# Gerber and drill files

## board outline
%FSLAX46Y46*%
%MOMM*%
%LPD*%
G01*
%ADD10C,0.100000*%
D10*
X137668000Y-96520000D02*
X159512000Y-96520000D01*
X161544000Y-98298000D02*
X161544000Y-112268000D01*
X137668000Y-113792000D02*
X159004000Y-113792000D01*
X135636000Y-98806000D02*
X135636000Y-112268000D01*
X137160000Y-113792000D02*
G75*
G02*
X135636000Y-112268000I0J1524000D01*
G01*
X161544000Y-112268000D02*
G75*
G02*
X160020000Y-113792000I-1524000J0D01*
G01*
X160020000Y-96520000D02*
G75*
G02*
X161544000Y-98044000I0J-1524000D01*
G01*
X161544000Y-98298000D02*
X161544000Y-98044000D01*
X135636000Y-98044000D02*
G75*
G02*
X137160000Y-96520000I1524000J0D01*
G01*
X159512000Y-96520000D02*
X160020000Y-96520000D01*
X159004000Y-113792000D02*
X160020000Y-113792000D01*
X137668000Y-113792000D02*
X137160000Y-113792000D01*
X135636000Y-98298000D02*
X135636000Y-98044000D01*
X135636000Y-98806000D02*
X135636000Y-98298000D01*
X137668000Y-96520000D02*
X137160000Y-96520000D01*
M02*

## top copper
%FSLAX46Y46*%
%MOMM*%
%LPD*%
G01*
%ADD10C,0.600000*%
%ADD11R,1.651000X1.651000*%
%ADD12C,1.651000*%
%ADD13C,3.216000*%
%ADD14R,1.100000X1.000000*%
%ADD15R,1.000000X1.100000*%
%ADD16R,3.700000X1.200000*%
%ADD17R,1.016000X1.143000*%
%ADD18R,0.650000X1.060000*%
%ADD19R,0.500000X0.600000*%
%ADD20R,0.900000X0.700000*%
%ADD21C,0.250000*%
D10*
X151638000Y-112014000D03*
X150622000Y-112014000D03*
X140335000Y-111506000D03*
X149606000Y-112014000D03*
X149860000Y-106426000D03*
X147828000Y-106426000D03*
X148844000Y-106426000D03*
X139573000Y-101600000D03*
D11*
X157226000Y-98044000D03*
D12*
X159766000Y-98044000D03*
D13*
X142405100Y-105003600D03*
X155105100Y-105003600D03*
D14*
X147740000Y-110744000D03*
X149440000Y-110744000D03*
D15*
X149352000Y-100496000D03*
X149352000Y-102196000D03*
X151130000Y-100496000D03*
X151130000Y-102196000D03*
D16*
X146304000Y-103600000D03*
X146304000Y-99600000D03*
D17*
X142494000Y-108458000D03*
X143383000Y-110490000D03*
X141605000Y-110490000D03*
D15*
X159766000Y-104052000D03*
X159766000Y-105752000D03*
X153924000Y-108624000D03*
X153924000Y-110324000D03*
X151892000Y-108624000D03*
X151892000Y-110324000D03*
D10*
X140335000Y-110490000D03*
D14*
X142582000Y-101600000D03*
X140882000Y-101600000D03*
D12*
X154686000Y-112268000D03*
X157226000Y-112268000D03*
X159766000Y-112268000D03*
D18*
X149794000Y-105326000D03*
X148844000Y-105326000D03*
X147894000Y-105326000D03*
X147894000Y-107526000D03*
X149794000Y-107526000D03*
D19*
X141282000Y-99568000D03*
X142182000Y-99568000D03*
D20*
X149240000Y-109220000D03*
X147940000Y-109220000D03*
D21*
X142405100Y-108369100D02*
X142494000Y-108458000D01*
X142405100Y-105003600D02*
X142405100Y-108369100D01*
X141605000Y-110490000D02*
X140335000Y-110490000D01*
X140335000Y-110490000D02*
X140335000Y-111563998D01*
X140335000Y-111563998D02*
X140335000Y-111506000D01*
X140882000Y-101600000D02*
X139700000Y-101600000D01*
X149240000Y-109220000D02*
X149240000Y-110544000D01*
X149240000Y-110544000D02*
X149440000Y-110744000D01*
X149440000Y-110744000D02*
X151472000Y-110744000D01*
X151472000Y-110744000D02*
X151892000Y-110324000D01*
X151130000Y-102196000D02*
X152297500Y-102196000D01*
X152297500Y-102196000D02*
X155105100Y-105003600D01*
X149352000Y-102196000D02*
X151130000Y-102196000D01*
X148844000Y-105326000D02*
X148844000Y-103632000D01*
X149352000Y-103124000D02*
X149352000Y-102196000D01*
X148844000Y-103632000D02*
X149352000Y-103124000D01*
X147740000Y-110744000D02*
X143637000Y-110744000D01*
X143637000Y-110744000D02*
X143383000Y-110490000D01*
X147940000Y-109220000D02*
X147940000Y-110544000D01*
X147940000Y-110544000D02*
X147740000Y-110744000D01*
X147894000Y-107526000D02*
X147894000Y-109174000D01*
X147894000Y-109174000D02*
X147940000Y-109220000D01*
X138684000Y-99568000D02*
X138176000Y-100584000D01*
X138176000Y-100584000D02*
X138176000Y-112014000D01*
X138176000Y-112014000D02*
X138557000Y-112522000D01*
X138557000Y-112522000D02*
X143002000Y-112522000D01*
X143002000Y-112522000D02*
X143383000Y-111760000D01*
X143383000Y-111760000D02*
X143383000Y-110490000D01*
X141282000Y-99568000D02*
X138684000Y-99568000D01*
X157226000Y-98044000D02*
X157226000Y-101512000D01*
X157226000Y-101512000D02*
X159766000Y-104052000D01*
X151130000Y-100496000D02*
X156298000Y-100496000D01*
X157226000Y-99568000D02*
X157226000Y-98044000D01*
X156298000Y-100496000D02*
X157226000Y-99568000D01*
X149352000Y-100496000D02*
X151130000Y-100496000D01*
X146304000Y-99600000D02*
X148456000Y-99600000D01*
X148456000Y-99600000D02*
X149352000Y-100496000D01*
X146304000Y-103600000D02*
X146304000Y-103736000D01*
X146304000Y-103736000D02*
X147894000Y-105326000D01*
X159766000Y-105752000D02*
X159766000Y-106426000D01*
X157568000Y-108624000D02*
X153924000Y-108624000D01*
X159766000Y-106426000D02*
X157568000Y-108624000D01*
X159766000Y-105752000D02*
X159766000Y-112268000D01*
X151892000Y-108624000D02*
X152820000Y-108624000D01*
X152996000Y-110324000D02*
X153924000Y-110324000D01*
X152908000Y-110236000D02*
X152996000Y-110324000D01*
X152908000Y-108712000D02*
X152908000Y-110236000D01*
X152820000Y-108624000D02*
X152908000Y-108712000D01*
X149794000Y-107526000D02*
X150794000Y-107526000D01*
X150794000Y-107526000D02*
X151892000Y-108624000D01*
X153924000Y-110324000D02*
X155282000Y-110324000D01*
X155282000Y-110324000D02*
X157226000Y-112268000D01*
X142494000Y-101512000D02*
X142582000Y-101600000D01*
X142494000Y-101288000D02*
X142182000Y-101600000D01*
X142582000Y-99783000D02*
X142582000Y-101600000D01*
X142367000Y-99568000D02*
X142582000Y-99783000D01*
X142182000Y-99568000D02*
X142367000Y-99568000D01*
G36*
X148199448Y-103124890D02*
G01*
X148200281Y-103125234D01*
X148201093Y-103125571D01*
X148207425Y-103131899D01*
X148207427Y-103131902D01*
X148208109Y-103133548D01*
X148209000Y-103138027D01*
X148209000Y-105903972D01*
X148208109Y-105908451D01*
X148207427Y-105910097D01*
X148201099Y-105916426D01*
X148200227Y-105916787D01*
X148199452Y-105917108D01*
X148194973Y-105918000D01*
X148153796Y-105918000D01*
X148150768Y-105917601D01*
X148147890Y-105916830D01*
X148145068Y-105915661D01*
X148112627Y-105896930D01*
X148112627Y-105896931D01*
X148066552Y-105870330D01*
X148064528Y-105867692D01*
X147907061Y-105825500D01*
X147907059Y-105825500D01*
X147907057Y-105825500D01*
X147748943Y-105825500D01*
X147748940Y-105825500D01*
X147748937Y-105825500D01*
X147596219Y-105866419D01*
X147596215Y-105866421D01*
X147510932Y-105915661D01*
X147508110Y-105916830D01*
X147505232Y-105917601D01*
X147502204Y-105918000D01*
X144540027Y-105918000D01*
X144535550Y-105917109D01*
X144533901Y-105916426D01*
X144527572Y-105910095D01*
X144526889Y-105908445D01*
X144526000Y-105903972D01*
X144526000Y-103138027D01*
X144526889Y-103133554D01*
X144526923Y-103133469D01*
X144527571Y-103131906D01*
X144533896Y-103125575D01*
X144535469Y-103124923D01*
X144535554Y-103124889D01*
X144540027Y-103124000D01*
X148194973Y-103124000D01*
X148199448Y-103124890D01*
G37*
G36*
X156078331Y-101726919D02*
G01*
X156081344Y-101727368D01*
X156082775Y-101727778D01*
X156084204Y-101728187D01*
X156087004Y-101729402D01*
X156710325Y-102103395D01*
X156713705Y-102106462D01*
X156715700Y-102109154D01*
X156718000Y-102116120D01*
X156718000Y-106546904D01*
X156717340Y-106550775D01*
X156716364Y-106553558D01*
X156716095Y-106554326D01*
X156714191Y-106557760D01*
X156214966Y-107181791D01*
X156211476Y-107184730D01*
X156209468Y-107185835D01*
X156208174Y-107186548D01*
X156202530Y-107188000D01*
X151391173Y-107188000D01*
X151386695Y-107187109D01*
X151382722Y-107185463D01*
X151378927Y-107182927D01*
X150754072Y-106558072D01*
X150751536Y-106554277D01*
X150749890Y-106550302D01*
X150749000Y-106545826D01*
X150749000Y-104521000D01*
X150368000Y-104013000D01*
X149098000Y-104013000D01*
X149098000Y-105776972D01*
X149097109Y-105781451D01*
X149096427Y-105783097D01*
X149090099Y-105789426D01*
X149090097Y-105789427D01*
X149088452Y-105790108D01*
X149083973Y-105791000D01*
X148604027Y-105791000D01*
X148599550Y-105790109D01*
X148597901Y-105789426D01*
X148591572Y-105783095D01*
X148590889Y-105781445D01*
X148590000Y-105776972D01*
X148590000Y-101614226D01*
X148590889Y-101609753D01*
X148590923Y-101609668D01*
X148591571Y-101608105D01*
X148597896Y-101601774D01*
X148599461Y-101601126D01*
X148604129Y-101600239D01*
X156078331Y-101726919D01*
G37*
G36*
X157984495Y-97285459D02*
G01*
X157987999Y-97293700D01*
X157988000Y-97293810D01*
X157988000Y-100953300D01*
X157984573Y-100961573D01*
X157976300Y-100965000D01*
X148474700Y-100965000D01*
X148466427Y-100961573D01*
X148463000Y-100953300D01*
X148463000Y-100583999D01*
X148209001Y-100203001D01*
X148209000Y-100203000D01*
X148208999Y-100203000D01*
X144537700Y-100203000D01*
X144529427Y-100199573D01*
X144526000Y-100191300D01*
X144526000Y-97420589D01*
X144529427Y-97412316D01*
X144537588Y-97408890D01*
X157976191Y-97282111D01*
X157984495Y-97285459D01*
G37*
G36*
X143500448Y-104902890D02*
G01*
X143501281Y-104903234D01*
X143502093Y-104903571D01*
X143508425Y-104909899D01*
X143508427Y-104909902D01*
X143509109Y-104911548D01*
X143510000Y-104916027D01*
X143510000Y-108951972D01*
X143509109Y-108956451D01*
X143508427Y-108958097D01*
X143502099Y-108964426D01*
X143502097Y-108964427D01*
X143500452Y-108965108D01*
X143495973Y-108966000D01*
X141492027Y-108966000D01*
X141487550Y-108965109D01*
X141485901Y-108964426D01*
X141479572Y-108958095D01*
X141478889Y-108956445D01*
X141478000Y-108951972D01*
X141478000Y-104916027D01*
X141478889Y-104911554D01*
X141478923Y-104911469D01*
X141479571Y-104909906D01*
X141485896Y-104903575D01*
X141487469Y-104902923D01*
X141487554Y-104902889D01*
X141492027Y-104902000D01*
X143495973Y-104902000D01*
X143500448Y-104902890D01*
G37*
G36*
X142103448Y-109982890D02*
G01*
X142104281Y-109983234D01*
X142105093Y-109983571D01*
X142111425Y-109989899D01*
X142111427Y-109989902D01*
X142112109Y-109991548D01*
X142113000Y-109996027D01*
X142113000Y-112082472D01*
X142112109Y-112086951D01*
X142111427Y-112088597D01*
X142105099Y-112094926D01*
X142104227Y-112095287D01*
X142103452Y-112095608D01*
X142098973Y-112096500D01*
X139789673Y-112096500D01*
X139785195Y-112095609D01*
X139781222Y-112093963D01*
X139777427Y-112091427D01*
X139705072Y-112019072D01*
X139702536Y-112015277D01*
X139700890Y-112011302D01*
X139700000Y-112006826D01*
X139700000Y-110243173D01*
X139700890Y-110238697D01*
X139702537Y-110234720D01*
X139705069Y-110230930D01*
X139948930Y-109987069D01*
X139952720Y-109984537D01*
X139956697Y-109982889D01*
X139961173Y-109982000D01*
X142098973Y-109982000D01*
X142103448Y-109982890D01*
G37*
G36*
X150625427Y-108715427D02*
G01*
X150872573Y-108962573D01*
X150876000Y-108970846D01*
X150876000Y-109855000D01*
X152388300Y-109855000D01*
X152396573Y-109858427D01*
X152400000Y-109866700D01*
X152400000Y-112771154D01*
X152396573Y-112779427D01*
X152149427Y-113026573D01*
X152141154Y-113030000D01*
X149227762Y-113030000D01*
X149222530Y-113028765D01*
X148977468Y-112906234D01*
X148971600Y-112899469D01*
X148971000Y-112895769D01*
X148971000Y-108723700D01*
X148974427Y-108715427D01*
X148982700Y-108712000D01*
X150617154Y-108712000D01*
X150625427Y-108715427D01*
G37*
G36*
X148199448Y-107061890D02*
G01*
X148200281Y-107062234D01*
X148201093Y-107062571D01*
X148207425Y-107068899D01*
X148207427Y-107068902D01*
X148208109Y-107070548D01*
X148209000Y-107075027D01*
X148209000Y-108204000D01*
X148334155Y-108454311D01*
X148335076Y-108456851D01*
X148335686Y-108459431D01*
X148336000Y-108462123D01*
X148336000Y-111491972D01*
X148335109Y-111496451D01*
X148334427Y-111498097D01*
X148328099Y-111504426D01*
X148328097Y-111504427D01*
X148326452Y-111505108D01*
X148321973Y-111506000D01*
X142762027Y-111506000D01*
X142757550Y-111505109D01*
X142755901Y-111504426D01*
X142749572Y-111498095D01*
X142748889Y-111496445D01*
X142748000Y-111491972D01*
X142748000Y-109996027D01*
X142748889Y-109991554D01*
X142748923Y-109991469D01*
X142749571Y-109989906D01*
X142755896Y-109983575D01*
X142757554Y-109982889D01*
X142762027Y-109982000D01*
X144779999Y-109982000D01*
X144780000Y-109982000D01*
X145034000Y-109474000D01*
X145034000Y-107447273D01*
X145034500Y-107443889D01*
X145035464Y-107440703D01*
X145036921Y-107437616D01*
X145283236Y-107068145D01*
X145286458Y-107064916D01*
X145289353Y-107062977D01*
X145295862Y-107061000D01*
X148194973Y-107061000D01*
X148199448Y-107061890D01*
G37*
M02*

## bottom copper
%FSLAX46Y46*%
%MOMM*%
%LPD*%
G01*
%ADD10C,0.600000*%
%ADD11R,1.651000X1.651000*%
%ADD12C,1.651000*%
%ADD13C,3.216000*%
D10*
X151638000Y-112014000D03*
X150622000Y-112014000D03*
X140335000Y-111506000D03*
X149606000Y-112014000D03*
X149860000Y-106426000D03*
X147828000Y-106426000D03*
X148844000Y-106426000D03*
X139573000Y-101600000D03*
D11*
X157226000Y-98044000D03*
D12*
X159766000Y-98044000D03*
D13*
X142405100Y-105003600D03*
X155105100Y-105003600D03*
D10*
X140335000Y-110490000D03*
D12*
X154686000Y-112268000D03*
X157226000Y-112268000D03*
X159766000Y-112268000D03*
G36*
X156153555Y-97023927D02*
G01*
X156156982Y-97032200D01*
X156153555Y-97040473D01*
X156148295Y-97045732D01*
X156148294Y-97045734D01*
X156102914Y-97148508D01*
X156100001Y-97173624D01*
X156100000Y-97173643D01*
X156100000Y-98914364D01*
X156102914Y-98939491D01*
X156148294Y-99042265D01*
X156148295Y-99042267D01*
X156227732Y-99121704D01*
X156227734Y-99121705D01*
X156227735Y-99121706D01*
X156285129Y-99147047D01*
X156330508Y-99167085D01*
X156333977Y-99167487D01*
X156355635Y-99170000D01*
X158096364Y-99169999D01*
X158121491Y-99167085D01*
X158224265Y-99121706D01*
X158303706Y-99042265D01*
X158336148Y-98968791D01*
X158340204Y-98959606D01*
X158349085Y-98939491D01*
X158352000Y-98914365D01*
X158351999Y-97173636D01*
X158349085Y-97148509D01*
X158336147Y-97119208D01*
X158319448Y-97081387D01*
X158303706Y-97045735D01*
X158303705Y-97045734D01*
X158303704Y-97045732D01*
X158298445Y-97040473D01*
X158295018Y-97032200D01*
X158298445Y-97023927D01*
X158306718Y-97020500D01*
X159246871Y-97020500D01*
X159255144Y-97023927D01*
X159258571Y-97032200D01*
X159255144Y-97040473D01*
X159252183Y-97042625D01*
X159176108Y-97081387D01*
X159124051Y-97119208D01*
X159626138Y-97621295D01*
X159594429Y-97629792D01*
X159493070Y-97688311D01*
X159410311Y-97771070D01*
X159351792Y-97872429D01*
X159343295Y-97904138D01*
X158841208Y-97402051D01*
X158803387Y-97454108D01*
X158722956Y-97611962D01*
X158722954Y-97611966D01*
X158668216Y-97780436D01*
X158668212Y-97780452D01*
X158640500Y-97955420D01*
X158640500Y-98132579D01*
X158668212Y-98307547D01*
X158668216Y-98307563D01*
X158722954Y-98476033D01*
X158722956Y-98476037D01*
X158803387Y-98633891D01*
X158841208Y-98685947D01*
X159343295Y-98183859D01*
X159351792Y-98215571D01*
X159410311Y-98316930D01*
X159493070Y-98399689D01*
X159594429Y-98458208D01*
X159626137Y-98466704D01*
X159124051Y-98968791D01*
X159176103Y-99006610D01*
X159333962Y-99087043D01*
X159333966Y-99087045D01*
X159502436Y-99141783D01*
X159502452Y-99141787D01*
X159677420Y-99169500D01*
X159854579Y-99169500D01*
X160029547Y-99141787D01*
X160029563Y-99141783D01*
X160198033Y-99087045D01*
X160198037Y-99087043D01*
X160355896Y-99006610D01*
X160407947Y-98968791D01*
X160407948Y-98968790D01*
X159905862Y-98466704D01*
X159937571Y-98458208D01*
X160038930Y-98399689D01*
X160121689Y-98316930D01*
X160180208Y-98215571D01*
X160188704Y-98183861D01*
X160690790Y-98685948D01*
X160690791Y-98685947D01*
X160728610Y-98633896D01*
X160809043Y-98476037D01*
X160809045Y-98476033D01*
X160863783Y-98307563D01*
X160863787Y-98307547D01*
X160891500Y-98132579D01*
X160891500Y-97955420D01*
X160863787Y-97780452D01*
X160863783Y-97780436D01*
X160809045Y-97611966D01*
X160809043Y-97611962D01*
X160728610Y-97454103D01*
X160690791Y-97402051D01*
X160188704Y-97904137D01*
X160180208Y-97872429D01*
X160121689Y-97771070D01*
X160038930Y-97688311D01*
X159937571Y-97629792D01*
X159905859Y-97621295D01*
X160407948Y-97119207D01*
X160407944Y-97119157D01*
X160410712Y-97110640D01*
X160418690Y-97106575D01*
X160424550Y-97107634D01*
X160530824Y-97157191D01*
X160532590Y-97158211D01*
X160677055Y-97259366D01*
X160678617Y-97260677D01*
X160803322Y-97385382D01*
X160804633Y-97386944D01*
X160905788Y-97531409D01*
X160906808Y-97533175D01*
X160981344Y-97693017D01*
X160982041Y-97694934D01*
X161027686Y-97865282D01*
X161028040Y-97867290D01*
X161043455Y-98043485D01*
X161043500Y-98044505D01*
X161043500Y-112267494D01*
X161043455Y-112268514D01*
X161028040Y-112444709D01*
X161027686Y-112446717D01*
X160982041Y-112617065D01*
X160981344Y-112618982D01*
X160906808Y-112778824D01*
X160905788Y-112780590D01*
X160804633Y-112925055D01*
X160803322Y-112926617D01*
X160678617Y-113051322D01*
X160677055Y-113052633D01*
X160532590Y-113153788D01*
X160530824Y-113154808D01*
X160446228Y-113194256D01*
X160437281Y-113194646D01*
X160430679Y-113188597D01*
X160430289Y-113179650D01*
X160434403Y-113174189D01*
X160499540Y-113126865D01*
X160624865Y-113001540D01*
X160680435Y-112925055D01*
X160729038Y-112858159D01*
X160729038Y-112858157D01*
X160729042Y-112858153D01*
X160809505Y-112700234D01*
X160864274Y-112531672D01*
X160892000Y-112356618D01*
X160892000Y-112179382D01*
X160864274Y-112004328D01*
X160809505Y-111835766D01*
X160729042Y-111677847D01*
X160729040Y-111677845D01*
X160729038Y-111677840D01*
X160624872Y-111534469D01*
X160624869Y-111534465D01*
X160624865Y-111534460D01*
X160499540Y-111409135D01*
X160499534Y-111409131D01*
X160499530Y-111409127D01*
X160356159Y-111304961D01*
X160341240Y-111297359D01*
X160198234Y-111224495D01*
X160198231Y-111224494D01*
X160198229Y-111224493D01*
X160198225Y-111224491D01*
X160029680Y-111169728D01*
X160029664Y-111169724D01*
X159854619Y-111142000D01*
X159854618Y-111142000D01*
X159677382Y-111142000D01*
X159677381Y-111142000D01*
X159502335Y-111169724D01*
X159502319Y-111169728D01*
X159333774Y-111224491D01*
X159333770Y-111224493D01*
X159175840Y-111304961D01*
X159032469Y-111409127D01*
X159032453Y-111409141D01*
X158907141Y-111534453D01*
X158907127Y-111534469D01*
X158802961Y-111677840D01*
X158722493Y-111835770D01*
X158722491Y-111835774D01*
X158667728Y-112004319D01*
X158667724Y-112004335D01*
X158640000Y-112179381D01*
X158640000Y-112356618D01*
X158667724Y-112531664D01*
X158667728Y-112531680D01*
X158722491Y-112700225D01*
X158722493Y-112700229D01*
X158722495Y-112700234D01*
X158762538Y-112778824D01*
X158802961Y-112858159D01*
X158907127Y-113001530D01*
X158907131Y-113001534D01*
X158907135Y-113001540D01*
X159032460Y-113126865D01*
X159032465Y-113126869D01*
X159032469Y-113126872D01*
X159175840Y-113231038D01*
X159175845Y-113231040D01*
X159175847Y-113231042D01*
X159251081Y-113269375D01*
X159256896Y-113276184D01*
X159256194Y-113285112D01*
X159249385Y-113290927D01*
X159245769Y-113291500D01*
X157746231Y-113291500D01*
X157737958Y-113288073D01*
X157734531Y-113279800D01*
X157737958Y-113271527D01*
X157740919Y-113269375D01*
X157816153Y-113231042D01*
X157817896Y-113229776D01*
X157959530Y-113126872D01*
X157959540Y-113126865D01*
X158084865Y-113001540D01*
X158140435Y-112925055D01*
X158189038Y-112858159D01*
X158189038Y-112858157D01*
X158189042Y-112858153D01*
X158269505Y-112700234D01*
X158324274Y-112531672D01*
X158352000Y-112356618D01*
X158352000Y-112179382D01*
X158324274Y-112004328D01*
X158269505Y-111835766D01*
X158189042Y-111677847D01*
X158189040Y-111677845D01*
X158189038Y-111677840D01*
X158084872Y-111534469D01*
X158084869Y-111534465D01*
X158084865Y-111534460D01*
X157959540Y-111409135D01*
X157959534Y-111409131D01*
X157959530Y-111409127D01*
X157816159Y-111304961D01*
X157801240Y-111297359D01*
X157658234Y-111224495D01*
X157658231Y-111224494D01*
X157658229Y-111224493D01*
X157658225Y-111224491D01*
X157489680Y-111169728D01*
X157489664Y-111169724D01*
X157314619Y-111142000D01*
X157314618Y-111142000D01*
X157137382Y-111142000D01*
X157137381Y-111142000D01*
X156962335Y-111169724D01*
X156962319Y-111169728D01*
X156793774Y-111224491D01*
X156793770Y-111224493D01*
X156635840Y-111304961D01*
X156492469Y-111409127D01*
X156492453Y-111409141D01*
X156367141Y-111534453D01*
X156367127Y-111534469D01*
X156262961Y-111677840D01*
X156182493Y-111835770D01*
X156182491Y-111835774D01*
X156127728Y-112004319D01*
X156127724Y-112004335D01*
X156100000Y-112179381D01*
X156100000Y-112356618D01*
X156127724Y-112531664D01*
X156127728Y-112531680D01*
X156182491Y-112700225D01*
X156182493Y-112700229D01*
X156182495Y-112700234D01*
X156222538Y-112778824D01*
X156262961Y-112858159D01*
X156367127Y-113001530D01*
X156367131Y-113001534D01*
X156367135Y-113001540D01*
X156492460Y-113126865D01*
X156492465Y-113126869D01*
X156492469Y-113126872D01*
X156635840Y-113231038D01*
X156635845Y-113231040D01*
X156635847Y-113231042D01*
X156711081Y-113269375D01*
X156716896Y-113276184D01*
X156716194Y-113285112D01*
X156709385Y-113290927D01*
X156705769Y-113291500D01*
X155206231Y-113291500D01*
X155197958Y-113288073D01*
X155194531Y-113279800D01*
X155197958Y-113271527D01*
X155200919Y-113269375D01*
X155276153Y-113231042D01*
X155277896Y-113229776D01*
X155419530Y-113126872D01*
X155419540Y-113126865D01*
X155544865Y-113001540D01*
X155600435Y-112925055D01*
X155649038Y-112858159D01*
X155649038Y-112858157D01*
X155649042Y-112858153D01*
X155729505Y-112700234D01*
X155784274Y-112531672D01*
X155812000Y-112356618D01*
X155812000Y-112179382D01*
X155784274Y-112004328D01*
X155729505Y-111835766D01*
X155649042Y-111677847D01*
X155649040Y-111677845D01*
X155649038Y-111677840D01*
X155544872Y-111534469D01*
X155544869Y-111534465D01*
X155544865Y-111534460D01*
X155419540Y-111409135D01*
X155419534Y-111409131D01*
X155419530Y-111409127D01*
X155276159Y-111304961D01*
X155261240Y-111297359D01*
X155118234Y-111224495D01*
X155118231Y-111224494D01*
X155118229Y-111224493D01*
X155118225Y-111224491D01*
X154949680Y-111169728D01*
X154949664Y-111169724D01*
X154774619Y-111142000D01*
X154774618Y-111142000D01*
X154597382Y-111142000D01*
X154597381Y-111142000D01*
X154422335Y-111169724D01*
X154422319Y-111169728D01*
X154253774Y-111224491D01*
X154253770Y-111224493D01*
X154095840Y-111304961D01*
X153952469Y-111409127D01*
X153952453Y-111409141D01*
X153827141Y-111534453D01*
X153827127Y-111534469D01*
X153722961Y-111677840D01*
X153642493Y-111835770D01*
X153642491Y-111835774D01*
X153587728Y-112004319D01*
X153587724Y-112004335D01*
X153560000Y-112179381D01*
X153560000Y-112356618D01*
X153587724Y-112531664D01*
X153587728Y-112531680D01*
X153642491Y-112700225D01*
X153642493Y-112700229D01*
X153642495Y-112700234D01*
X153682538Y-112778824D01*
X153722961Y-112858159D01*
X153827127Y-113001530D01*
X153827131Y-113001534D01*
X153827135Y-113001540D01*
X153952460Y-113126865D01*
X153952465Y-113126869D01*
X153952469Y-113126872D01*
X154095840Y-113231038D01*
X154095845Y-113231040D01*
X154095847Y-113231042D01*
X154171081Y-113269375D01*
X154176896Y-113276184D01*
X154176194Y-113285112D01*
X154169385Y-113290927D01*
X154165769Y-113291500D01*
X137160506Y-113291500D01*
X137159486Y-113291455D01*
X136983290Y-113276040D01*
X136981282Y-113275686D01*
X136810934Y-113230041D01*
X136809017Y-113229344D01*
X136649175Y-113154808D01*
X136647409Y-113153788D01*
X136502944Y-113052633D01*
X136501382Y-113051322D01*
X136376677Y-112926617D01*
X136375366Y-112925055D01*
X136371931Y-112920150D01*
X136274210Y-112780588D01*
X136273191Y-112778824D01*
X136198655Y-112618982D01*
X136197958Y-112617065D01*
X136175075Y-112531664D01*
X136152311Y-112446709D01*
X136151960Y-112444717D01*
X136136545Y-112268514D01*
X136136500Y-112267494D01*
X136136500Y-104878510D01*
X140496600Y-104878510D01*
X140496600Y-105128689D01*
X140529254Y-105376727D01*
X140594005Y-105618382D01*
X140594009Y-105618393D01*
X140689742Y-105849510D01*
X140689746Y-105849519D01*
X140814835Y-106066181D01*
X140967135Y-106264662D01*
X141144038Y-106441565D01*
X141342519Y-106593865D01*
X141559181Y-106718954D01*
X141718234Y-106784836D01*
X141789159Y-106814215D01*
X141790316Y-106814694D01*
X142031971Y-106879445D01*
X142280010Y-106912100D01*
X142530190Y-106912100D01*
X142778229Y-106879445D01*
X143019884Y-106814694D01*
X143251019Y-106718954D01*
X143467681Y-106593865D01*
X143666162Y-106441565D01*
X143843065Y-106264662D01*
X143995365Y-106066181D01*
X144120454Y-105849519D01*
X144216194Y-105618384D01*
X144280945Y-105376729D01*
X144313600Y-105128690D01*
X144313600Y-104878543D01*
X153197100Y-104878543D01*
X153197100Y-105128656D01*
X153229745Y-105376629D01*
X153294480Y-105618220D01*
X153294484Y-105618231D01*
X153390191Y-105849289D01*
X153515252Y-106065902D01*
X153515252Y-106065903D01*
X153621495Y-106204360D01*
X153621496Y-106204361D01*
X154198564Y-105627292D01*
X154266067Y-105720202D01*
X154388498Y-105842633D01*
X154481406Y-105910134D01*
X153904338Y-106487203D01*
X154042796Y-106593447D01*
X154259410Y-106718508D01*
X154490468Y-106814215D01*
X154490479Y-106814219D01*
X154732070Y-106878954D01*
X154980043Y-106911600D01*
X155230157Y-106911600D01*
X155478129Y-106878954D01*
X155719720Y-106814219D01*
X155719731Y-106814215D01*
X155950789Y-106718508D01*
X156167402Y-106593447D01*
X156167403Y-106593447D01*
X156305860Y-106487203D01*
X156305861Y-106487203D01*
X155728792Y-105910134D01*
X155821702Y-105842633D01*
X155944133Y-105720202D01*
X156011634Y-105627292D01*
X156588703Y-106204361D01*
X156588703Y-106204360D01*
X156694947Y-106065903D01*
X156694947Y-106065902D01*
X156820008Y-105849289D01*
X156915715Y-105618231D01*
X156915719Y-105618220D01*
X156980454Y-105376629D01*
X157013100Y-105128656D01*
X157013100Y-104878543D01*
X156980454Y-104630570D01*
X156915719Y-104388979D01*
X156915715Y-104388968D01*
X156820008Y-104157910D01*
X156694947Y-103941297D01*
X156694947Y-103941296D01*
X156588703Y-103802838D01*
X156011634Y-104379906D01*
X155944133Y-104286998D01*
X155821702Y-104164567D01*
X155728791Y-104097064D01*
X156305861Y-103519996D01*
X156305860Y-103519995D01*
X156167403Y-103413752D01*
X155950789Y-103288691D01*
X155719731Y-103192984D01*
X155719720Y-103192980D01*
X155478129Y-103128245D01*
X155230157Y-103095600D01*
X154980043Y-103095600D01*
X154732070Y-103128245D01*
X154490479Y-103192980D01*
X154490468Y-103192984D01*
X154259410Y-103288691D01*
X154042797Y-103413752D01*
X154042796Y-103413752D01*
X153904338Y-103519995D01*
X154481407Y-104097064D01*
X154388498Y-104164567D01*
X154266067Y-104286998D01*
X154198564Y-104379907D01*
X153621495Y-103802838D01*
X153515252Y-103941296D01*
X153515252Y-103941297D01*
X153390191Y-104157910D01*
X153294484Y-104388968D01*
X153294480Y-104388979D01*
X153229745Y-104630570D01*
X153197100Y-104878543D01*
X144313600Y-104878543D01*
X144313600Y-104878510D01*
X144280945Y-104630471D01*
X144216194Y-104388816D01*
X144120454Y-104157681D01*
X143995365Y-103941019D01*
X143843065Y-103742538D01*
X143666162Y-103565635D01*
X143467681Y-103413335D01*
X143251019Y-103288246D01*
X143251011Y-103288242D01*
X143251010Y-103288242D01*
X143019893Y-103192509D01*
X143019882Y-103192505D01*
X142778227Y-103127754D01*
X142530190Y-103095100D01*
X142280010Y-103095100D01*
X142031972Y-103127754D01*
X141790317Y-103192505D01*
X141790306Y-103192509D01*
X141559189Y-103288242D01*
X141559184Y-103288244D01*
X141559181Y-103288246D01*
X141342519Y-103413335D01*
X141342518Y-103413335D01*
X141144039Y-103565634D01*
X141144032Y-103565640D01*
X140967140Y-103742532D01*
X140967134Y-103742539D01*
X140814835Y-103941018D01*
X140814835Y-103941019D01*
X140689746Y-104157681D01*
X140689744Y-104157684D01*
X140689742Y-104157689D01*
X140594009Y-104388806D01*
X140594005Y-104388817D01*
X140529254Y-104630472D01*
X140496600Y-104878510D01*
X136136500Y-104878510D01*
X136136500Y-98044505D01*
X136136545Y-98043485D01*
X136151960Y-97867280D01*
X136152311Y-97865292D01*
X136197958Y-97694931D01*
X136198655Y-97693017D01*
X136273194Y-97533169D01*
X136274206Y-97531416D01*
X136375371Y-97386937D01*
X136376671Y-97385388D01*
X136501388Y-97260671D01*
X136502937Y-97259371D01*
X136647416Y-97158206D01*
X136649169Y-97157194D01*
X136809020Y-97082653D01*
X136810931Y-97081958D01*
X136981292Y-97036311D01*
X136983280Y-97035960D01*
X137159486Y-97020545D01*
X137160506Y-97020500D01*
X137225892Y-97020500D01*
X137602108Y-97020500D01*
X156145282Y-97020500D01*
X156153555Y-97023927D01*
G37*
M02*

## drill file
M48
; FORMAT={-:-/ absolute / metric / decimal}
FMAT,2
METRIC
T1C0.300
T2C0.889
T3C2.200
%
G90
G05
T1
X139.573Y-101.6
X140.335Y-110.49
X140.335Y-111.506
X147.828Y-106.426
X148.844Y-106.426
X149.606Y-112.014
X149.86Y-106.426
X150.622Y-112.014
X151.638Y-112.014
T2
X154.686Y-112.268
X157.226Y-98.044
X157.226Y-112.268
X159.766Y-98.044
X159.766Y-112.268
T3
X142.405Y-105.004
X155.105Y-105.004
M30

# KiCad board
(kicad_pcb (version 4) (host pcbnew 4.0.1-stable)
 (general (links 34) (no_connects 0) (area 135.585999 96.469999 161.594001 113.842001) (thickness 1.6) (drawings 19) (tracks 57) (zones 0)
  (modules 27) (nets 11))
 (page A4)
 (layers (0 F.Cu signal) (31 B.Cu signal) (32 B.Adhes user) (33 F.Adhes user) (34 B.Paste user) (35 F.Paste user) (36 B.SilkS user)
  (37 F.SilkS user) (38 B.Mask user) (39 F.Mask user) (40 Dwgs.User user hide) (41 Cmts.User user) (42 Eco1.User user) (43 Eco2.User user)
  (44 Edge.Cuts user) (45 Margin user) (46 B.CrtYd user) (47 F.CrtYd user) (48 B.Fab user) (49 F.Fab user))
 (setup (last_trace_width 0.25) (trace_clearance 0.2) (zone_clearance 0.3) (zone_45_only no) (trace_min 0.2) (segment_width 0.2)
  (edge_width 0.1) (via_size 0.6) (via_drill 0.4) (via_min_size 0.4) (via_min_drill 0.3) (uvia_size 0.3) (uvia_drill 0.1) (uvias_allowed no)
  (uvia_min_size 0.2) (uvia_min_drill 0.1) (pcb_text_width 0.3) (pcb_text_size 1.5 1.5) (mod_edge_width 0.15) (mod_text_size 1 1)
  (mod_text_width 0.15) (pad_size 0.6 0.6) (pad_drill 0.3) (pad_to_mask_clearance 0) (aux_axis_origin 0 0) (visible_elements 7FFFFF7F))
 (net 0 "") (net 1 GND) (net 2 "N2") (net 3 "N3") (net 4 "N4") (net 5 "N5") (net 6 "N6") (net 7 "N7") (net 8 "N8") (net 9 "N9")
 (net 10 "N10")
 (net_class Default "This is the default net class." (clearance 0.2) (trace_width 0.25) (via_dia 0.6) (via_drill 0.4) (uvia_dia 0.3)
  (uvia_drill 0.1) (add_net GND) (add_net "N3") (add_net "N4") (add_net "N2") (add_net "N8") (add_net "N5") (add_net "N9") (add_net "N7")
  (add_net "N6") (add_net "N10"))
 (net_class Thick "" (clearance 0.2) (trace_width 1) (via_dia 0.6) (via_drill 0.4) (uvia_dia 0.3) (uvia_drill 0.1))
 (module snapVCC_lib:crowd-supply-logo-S (layer F.Cu) (at 138 98.15 90)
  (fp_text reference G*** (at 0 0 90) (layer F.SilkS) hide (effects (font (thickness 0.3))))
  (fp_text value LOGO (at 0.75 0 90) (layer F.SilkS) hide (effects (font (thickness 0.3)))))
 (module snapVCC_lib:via (layer F.Cu) (at 151.638 112.014)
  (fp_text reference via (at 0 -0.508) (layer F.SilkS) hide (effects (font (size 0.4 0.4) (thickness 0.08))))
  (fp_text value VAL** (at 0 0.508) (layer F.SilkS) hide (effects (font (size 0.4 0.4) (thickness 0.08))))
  (pad 1 thru_hole circle (at 0 0) (size 0.6 0.6) (drill 0.3) (layers *.Cu) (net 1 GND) (zone_connect 2)))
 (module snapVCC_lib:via (layer F.Cu) (at 150.622 112.014)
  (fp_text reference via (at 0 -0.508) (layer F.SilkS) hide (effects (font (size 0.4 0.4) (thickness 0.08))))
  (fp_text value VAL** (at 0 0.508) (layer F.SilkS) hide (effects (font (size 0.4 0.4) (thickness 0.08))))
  (pad 1 thru_hole circle (at 0 0) (size 0.6 0.6) (drill 0.3) (layers *.Cu) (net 1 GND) (zone_connect 2)))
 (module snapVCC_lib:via (layer F.Cu) (at 140.335 111.506)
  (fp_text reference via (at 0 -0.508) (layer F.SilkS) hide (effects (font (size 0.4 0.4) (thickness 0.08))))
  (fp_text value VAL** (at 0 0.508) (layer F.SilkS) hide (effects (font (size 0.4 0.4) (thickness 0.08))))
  (pad 1 thru_hole circle (at 0 0) (size 0.6 0.6) (drill 0.3) (layers *.Cu) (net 1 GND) (zone_connect 2)))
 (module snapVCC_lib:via (layer F.Cu) (at 149.606 112.014)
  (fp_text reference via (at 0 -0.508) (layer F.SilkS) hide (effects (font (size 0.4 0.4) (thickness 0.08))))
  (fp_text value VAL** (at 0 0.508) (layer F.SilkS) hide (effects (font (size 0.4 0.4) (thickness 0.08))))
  (pad 1 thru_hole circle (at 0 0) (size 0.6 0.6) (drill 0.3) (layers *.Cu) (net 1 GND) (zone_connect 2)))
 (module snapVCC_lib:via (layer F.Cu) (at 149.86 106.426)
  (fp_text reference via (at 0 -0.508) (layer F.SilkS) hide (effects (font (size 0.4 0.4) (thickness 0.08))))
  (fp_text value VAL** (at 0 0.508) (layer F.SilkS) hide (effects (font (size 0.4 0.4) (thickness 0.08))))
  (pad 1 thru_hole circle (at 0 0) (size 0.6 0.6) (drill 0.3) (layers *.Cu) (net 1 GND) (zone_connect 2)))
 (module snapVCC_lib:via (layer F.Cu) (at 147.828 106.426)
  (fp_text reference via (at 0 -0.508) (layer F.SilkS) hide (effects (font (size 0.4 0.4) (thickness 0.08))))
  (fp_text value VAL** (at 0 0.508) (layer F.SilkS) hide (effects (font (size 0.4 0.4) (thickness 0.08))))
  (pad 1 thru_hole circle (at 0 0) (size 0.6 0.6) (drill 0.3) (layers *.Cu) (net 1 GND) (zone_connect 2)))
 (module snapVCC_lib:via (layer F.Cu) (at 148.844 106.426)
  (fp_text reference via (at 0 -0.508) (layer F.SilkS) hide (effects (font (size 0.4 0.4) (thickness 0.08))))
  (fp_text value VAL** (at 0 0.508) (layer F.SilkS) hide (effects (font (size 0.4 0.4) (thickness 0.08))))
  (pad 1 thru_hole circle (at 0 0) (size 0.6 0.6) (drill 0.3) (layers *.Cu) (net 1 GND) (zone_connect 2)))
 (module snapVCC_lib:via (layer F.Cu) (at 139.573 101.6)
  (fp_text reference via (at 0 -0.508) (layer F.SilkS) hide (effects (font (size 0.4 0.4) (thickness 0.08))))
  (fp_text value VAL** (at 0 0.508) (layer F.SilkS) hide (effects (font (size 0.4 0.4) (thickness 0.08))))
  (pad 1 thru_hole circle (at 0 0) (size 0.6 0.6) (drill 0.3) (layers *.Cu) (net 1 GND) (zone_connect 2)))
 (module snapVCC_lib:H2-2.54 (layer F.Cu) (at 158.496 98.044 90)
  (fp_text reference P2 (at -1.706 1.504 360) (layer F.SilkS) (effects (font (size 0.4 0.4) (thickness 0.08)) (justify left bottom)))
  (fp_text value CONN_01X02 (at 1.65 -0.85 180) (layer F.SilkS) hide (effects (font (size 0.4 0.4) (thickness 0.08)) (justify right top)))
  (pad 1 thru_hole rect (at 0 -1.27 90) (size 1.651 1.651) (drill 0.889) (layers *.Cu *.Mask) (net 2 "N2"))
  (pad 2 thru_hole circle (at 0 1.27 90) (size 1.651 1.651) (drill 0.889) (layers *.Cu *.Mask) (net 1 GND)))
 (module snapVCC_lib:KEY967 (layer B.Cu) (at 148.7551 105.0036)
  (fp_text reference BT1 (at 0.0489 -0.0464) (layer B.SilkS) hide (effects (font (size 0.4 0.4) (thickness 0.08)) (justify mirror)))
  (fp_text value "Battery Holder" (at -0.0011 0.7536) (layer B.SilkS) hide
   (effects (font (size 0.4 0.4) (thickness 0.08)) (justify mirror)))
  (pad 1 thru_hole circle (at -6.35 0) (size 3.216 3.216) (drill 2.2) (layers *.Cu *.Mask) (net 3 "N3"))
  (pad 2 thru_hole circle (at 6.35 0) (size 3.216 3.216) (drill 2.2) (layers *.Cu *.Mask) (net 1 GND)))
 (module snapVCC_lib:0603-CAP (layer F.Cu) (at 148.59 110.744)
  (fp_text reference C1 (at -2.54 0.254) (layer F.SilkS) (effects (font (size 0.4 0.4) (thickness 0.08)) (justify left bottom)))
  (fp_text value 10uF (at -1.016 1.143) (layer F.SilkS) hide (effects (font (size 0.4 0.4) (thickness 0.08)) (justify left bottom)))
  (pad 1 smd rect (at -0.85 0) (size 1.1 1) (layers F.Cu F.Paste F.Mask) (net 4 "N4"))
  (pad 2 smd rect (at 0.85 0) (size 1.1 1) (layers F.Cu F.Paste F.Mask) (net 1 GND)))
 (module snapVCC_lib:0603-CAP (layer F.Cu) (at 149.352 101.346 270)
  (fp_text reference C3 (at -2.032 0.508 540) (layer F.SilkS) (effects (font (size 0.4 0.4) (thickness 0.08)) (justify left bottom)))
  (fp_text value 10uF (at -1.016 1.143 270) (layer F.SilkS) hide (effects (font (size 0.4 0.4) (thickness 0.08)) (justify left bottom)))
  (pad 1 smd rect (at -0.85 0 270) (size 1.1 1) (layers F.Cu F.Paste F.Mask) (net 2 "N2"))
  (pad 2 smd rect (at 0.85 0 270) (size 1.1 1) (layers F.Cu F.Paste F.Mask) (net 1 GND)))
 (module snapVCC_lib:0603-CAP (layer F.Cu) (at 151.13 101.346 270)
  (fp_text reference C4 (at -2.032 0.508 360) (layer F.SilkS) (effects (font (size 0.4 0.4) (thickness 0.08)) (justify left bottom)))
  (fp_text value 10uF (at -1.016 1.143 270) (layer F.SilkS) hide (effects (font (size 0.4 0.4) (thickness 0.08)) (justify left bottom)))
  (pad 1 smd rect (at -0.85 0 270) (size 1.1 1) (layers F.Cu F.Paste F.Mask) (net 2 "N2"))
  (pad 2 smd rect (at 0.85 0 270) (size 1.1 1) (layers F.Cu F.Paste F.Mask) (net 1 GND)))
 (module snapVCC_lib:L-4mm (layer F.Cu) (at 146.304 101.6 90)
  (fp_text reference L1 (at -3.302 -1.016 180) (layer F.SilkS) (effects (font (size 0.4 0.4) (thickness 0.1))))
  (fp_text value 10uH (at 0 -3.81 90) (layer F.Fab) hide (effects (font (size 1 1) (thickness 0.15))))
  (pad 1 smd rect (at -2 0 90) (size 1.2 3.7) (layers F.Cu F.Paste F.Mask) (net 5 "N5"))
  (pad 2 smd rect (at 2 0 90) (size 1.2 3.7) (layers F.Cu F.Paste F.Mask) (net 2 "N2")))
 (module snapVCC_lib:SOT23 (layer F.Cu) (at 142.494 109.474)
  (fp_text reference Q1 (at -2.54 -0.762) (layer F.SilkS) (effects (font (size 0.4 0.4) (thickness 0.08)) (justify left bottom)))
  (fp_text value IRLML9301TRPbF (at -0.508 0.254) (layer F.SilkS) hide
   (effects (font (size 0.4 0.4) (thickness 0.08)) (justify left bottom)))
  (pad 3 smd rect (at 0 -1.016) (size 1.016 1.143) (layers F.Cu F.Paste F.Mask) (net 3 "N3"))
  (pad 2 smd rect (at 0.889 1.016) (size 1.016 1.143) (layers F.Cu F.Paste F.Mask) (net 4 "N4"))
  (pad 1 smd rect (at -0.889 1.016 180) (size 1.016 1.143) (layers F.Cu F.Paste F.Mask) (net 1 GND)))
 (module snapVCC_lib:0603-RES (layer F.Cu) (at 159.766 104.902 270)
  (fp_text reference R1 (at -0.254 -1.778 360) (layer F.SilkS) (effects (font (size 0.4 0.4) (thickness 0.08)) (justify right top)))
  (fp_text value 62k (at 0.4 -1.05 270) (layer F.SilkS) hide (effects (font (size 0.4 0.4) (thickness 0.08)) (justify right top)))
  (pad 1 smd rect (at -0.85 0 270) (size 1.1 1) (layers F.Cu F.Paste F.Mask) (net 2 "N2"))
  (pad 2 smd rect (at 0.85 0 270) (size 1.1 1) (layers F.Cu F.Paste F.Mask) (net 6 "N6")))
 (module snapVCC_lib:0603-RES (layer F.Cu) (at 153.924 109.474 270)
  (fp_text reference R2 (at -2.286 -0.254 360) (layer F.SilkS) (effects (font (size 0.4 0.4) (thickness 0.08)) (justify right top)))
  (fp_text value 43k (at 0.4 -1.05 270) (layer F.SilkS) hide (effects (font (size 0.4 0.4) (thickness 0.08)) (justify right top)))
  (pad 1 smd rect (at -0.85 0 270) (size 1.1 1) (layers F.Cu F.Paste F.Mask) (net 6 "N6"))
  (pad 2 smd rect (at 0.85 0 270) (size 1.1 1) (layers F.Cu F.Paste F.Mask) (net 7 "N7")))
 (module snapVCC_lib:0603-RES (layer F.Cu) (at 151.892 109.474 270)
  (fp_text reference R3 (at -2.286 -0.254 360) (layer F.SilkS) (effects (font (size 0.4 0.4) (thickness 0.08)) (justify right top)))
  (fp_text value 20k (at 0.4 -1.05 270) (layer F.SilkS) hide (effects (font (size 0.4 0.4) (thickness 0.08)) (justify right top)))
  (pad 1 smd rect (at -0.85 0 270) (size 1.1 1) (layers F.Cu F.Paste F.Mask) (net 7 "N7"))
  (pad 2 smd rect (at 0.85 0 270) (size 1.1 1) (layers F.Cu F.Paste F.Mask) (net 1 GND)))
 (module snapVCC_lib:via (layer F.Cu) (at 140.335 110.49)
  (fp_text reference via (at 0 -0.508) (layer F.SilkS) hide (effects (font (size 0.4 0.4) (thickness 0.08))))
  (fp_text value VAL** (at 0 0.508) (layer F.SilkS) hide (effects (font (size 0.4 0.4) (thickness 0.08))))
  (pad 1 thru_hole circle (at 0 0) (size 0.6 0.6) (drill 0.3) (layers *.Cu) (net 1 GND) (zone_connect 2)))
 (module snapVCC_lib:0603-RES (layer F.Cu) (at 141.732 101.6 180)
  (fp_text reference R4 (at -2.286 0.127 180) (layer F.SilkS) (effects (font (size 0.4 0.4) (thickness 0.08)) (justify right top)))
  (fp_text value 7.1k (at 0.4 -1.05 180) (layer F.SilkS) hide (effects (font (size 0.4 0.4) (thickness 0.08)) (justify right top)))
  (pad 1 smd rect (at -0.85 0 180) (size 1.1 1) (layers F.Cu F.Paste F.Mask) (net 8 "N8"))
  (pad 2 smd rect (at 0.85 0 180) (size 1.1 1) (layers F.Cu F.Paste F.Mask) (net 1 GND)))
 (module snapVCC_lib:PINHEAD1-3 (layer F.Cu) (at 157.226 112.268)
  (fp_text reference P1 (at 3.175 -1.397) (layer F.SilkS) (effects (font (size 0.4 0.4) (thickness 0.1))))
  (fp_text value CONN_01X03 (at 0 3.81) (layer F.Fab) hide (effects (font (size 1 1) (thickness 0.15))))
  (pad 1 thru_hole circle (at -2.54 0) (size 1.651 1.651) (drill 0.889) (layers *.Cu *.Mask) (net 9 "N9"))
  (pad 2 thru_hole circle (at 0 0) (size 1.651 1.651) (drill 0.889) (layers *.Cu *.Mask) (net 7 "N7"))
  (pad 3 thru_hole circle (at 2.54 0) (size 1.651 1.651) (drill 0.889) (layers *.Cu *.Mask) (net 6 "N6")))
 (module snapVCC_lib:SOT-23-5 (layer F.Cu) (at 148.844 106.426 270)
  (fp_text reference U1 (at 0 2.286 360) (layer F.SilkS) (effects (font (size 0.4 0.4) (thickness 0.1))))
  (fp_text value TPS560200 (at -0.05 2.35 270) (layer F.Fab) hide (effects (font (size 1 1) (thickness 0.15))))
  (pad 1 smd rect (at -1.1 -0.95 270) (size 1.06 0.65) (layers F.Cu F.Paste F.Mask) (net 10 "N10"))
  (pad 2 smd rect (at -1.1 0 270) (size 1.06 0.65) (layers F.Cu F.Paste F.Mask) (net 1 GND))
  (pad 3 smd rect (at -1.1 0.95 270) (size 1.06 0.65) (layers F.Cu F.Paste F.Mask) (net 5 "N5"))
  (pad 4 smd rect (at 1.1 0.95 270) (size 1.06 0.65) (layers F.Cu F.Paste F.Mask) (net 4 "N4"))
  (pad 5 smd rect (at 1.1 -0.95 270) (size 1.06 0.65) (layers F.Cu F.Paste F.Mask) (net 7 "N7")))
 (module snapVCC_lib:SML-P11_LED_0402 (layer F.Cu) (at 141.732 99.568 180)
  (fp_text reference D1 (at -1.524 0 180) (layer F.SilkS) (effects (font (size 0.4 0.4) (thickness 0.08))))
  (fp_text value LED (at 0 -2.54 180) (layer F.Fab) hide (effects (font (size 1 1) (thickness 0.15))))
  (pad 2 smd rect (at 0.45 0 180) (size 0.5 0.6) (layers F.Cu F.Paste F.Mask) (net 4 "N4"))
  (pad 1 smd rect (at -0.45 0 180) (size 0.5 0.6) (layers F.Cu F.Paste F.Mask) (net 8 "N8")))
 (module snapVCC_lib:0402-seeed (layer F.Cu) (at 148.59 109.22)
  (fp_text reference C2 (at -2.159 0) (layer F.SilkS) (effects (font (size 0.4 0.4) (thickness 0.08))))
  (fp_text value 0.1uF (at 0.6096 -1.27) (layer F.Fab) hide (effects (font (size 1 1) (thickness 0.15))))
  (pad 2 smd rect (at 0.65 0) (size 0.9 0.7) (layers F.Cu F.Paste F.Mask) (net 1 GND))
  (pad 1 smd rect (at -0.65 0) (size 0.9 0.7) (layers F.Cu F.Paste F.Mask) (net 4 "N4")))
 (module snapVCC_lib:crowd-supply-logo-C (layer F.Cu) (at 138 99.85 90)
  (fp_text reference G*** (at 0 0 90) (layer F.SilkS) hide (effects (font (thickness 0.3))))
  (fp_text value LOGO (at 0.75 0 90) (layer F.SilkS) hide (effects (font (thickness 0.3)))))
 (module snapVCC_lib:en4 (layer F.Cu) (at 137.85 107.6 90)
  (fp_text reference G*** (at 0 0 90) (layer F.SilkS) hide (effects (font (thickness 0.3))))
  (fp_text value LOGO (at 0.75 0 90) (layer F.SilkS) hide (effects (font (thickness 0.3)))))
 (gr_line (start 137.668 96.52) (end 159.512 96.52) (angle 90) (layer Edge.Cuts) (width 0.1))
 (gr_line (start 161.544 98.298) (end 161.544 112.268) (angle 90) (layer Edge.Cuts) (width 0.1))
 (gr_line (start 137.668 113.792) (end 159.004 113.792) (angle 90) (layer Edge.Cuts) (width 0.1))
 (gr_line (start 135.636 98.806) (end 135.636 112.268) (angle 90) (layer Edge.Cuts) (width 0.1))
 (gr_arc (start 137.16 112.268) (end 137.16 113.792) (angle 90) (layer Edge.Cuts) (width 0.1))
 (gr_arc (start 160.02 112.268) (end 161.544 112.268) (angle 90) (layer Edge.Cuts) (width 0.1))
 (gr_arc (start 160.02 98.044) (end 160.02 96.52) (angle 90) (layer Edge.Cuts) (width 0.1))
 (gr_line (start 161.544 98.298) (end 161.544 98.044) (angle 90) (layer Edge.Cuts) (width 0.1))
 (gr_arc (start 137.16 98.044) (end 135.636 98.044) (angle 90) (layer Edge.Cuts) (width 0.1))
 (gr_line (start 159.512 96.52) (end 160.02 96.52) (angle 90) (layer Edge.Cuts) (width 0.1))
 (gr_line (start 159.004 113.792) (end 160.02 113.792) (angle 90) (layer Edge.Cuts) (width 0.1))
 (gr_line (start 137.668 113.792) (end 137.16 113.792) (angle 90) (layer Edge.Cuts) (width 0.1))
 (gr_line (start 135.636 98.298) (end 135.636 98.044) (angle 90) (layer Edge.Cuts) (width 0.1))
 (gr_line (start 135.636 98.806) (end 135.636 98.298) (angle 90) (layer Edge.Cuts) (width 0.1))
 (gr_line (start 137.668 96.52) (end 137.16 96.52) (angle 90) (layer Edge.Cuts) (width 0.1))
 (segment (start 142.4051 108.3691) (end 142.494 108.458) (width 0.25) (layer F.Cu) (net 3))
 (segment (start 142.4051 105.0036) (end 142.4051 108.3691) (width 0.25) (layer F.Cu) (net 3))
 (segment (start 141.605 110.49) (end 140.335 110.49) (width 0.25) (layer F.Cu) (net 1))
 (segment (start 140.335 110.49) (end 140.335 111.563998) (width 0.25) (layer F.Cu) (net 1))
 (segment (start 140.335 111.563998) (end 140.335 111.506) (width 0.25) (layer F.Cu) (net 1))
 (segment (start 140.882 101.6) (end 139.7 101.6) (width 0.25) (layer F.Cu) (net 1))
 (segment (start 149.24 109.22) (end 149.24 110.544) (width 0.25) (layer F.Cu) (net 1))
 (segment (start 149.24 110.544) (end 149.44 110.744) (width 0.25) (layer F.Cu) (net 1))
 (segment (start 149.44 110.744) (end 151.472 110.744) (width 0.25) (layer F.Cu) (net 1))
 (segment (start 151.472 110.744) (end 151.892 110.324) (width 0.25) (layer F.Cu) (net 1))
 (segment (start 151.13 102.196) (end 152.2975 102.196) (width 0.25) (layer F.Cu) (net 1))
 (segment (start 152.2975 102.196) (end 155.1051 105.0036) (width 0.25) (layer F.Cu) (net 1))
 (segment (start 149.352 102.196) (end 151.13 102.196) (width 0.25) (layer F.Cu) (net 1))
 (segment (start 148.844 105.326) (end 148.844 103.632) (width 0.25) (layer F.Cu) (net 1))
 (segment (start 149.352 103.124) (end 149.352 102.196) (width 0.25) (layer F.Cu) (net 1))
 (segment (start 148.844 103.632) (end 149.352 103.124) (width 0.25) (layer F.Cu) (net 1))
 (segment (start 147.74 110.744) (end 143.637 110.744) (width 0.25) (layer F.Cu) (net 4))
 (segment (start 143.637 110.744) (end 143.383 110.49) (width 0.25) (layer F.Cu) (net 4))
 (segment (start 147.94 109.22) (end 147.94 110.544) (width 0.25) (layer F.Cu) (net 4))
 (segment (start 147.94 110.544) (end 147.74 110.744) (width 0.25) (layer F.Cu) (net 4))
 (segment (start 147.894 107.526) (end 147.894 109.174) (width 0.25) (layer F.Cu) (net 4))
 (segment (start 147.894 109.174) (end 147.94 109.22) (width 0.25) (layer F.Cu) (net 4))
 (segment (start 138.684 99.568) (end 138.176 100.584) (width 0.25) (layer F.Cu) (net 4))
 (segment (start 138.176 100.584) (end 138.176 112.014) (width 0.25) (layer F.Cu) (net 4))
 (segment (start 138.176 112.014) (end 138.557 112.522) (width 0.25) (layer F.Cu) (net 4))
 (segment (start 138.557 112.522) (end 143.002 112.522) (width 0.25) (layer F.Cu) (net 4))
 (segment (start 143.002 112.522) (end 143.383 111.76) (width 0.25) (layer F.Cu) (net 4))
 (segment (start 143.383 111.76) (end 143.383 110.49) (width 0.25) (layer F.Cu) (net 4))
 (segment (start 141.282 99.568) (end 138.684 99.568) (width 0.25) (layer F.Cu) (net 4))
 (segment (start 157.226 98.044) (end 157.226 101.512) (width 0.25) (layer F.Cu) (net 2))
 (segment (start 157.226 101.512) (end 159.766 104.052) (width 0.25) (layer F.Cu) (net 2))
 (segment (start 151.13 100.496) (end 156.298 100.496) (width 0.25) (layer F.Cu) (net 2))
 (segment (start 157.226 99.568) (end 157.226 98.044) (width 0.25) (layer F.Cu) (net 2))
 (segment (start 156.298 100.496) (end 157.226 99.568) (width 0.25) (layer F.Cu) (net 2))
 (segment (start 149.352 100.496) (end 151.13 100.496) (width 0.25) (layer F.Cu) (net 2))
 (segment (start 146.304 99.6) (end 148.456 99.6) (width 0.25) (layer F.Cu) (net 2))
 (segment (start 148.456 99.6) (end 149.352 100.496) (width 0.25) (layer F.Cu) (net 2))
 (segment (start 146.304 103.6) (end 146.304 103.736) (width 0.25) (layer F.Cu) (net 5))
 (segment (start 146.304 103.736) (end 147.894 105.326) (width 0.25) (layer F.Cu) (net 5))
 (segment (start 159.766 105.752) (end 159.766 106.426) (width 0.25) (layer F.Cu) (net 6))
 (segment (start 157.568 108.624) (end 153.924 108.624) (width 0.25) (layer F.Cu) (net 6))
 (segment (start 159.766 106.426) (end 157.568 108.624) (width 0.25) (layer F.Cu) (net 6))
 (segment (start 159.766 105.752) (end 159.766 112.268) (width 0.25) (layer F.Cu) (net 6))
 (segment (start 151.892 108.624) (end 152.82 108.624) (width 0.25) (layer F.Cu) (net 7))
 (segment (start 152.996 110.324) (end 153.924 110.324) (width 0.25) (layer F.Cu) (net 7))
 (segment (start 152.908 110.236) (end 152.996 110.324) (width 0.25) (layer F.Cu) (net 7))
 (segment (start 152.908 108.712) (end 152.908 110.236) (width 0.25) (layer F.Cu) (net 7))
 (segment (start 152.82 108.624) (end 152.908 108.712) (width 0.25) (layer F.Cu) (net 7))
 (segment (start 149.794 107.526) (end 150.794 107.526) (width 0.25) (layer F.Cu) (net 7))
 (segment (start 150.794 107.526) (end 151.892 108.624) (width 0.25) (layer F.Cu) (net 7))
 (segment (start 153.924 110.324) (end 155.282 110.324) (width 0.25) (layer F.Cu) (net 7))
 (segment (start 155.282 110.324) (end 157.226 112.268) (width 0.25) (layer F.Cu) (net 7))
 (segment (start 142.494 101.512) (end 142.582 101.6) (width 0.25) (layer F.Cu) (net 8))
 (segment (start 142.494 101.288) (end 142.182 101.6) (width 0.25) (layer F.Cu) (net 8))
 (segment (start 142.582 99.783) (end 142.582 101.6) (width 0.25) (layer F.Cu) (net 8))
 (segment (start 142.367 99.568) (end 142.582 99.783) (width 0.25) (layer F.Cu) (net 8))
 (segment (start 142.182 99.568) (end 142.367 99.568) (width 0.25) (layer F.Cu) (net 8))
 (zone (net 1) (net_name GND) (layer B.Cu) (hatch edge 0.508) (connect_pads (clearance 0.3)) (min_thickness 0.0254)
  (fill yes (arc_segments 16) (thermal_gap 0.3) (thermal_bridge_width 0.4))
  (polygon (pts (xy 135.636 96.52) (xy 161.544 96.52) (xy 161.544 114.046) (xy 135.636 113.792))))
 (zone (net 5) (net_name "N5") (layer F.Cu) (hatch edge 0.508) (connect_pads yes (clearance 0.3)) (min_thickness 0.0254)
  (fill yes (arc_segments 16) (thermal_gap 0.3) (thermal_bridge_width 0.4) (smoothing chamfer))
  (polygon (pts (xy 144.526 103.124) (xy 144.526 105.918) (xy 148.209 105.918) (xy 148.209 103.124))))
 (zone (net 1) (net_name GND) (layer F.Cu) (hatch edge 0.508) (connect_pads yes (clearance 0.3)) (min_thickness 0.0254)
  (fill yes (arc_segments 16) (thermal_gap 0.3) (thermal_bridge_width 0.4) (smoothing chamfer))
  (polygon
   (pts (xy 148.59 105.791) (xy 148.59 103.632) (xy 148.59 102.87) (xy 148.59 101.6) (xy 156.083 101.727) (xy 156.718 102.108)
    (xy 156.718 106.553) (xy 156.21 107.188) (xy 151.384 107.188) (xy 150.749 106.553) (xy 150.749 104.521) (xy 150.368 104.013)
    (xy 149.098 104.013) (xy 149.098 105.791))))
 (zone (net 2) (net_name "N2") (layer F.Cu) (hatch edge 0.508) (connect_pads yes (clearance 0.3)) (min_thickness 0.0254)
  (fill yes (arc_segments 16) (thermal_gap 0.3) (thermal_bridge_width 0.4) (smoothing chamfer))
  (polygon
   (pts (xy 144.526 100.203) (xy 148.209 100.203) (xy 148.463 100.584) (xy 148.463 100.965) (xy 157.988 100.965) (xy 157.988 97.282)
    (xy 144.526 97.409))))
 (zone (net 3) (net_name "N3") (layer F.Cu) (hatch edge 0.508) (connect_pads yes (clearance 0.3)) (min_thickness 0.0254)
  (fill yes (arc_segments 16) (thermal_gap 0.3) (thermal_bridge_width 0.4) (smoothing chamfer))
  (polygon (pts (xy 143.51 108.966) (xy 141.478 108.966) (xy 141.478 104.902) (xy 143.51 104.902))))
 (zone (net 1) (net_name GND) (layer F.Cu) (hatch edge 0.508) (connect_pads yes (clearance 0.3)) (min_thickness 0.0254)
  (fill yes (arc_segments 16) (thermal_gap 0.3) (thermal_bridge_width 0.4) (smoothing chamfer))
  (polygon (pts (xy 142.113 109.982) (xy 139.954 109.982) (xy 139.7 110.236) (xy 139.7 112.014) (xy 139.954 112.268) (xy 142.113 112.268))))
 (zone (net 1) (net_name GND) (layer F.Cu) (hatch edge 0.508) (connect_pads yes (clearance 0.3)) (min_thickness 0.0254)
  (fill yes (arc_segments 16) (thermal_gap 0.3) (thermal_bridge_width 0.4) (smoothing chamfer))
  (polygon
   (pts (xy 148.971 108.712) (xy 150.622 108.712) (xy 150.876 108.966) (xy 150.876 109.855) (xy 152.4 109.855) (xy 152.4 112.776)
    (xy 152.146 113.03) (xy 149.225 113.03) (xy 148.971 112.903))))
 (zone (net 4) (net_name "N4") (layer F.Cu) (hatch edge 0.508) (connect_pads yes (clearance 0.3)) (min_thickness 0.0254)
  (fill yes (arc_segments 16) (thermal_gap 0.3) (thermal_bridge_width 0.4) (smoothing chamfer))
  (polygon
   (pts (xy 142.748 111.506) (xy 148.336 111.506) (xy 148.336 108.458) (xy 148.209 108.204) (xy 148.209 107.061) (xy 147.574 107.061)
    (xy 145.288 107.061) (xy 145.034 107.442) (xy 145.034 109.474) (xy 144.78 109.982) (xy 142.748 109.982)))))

